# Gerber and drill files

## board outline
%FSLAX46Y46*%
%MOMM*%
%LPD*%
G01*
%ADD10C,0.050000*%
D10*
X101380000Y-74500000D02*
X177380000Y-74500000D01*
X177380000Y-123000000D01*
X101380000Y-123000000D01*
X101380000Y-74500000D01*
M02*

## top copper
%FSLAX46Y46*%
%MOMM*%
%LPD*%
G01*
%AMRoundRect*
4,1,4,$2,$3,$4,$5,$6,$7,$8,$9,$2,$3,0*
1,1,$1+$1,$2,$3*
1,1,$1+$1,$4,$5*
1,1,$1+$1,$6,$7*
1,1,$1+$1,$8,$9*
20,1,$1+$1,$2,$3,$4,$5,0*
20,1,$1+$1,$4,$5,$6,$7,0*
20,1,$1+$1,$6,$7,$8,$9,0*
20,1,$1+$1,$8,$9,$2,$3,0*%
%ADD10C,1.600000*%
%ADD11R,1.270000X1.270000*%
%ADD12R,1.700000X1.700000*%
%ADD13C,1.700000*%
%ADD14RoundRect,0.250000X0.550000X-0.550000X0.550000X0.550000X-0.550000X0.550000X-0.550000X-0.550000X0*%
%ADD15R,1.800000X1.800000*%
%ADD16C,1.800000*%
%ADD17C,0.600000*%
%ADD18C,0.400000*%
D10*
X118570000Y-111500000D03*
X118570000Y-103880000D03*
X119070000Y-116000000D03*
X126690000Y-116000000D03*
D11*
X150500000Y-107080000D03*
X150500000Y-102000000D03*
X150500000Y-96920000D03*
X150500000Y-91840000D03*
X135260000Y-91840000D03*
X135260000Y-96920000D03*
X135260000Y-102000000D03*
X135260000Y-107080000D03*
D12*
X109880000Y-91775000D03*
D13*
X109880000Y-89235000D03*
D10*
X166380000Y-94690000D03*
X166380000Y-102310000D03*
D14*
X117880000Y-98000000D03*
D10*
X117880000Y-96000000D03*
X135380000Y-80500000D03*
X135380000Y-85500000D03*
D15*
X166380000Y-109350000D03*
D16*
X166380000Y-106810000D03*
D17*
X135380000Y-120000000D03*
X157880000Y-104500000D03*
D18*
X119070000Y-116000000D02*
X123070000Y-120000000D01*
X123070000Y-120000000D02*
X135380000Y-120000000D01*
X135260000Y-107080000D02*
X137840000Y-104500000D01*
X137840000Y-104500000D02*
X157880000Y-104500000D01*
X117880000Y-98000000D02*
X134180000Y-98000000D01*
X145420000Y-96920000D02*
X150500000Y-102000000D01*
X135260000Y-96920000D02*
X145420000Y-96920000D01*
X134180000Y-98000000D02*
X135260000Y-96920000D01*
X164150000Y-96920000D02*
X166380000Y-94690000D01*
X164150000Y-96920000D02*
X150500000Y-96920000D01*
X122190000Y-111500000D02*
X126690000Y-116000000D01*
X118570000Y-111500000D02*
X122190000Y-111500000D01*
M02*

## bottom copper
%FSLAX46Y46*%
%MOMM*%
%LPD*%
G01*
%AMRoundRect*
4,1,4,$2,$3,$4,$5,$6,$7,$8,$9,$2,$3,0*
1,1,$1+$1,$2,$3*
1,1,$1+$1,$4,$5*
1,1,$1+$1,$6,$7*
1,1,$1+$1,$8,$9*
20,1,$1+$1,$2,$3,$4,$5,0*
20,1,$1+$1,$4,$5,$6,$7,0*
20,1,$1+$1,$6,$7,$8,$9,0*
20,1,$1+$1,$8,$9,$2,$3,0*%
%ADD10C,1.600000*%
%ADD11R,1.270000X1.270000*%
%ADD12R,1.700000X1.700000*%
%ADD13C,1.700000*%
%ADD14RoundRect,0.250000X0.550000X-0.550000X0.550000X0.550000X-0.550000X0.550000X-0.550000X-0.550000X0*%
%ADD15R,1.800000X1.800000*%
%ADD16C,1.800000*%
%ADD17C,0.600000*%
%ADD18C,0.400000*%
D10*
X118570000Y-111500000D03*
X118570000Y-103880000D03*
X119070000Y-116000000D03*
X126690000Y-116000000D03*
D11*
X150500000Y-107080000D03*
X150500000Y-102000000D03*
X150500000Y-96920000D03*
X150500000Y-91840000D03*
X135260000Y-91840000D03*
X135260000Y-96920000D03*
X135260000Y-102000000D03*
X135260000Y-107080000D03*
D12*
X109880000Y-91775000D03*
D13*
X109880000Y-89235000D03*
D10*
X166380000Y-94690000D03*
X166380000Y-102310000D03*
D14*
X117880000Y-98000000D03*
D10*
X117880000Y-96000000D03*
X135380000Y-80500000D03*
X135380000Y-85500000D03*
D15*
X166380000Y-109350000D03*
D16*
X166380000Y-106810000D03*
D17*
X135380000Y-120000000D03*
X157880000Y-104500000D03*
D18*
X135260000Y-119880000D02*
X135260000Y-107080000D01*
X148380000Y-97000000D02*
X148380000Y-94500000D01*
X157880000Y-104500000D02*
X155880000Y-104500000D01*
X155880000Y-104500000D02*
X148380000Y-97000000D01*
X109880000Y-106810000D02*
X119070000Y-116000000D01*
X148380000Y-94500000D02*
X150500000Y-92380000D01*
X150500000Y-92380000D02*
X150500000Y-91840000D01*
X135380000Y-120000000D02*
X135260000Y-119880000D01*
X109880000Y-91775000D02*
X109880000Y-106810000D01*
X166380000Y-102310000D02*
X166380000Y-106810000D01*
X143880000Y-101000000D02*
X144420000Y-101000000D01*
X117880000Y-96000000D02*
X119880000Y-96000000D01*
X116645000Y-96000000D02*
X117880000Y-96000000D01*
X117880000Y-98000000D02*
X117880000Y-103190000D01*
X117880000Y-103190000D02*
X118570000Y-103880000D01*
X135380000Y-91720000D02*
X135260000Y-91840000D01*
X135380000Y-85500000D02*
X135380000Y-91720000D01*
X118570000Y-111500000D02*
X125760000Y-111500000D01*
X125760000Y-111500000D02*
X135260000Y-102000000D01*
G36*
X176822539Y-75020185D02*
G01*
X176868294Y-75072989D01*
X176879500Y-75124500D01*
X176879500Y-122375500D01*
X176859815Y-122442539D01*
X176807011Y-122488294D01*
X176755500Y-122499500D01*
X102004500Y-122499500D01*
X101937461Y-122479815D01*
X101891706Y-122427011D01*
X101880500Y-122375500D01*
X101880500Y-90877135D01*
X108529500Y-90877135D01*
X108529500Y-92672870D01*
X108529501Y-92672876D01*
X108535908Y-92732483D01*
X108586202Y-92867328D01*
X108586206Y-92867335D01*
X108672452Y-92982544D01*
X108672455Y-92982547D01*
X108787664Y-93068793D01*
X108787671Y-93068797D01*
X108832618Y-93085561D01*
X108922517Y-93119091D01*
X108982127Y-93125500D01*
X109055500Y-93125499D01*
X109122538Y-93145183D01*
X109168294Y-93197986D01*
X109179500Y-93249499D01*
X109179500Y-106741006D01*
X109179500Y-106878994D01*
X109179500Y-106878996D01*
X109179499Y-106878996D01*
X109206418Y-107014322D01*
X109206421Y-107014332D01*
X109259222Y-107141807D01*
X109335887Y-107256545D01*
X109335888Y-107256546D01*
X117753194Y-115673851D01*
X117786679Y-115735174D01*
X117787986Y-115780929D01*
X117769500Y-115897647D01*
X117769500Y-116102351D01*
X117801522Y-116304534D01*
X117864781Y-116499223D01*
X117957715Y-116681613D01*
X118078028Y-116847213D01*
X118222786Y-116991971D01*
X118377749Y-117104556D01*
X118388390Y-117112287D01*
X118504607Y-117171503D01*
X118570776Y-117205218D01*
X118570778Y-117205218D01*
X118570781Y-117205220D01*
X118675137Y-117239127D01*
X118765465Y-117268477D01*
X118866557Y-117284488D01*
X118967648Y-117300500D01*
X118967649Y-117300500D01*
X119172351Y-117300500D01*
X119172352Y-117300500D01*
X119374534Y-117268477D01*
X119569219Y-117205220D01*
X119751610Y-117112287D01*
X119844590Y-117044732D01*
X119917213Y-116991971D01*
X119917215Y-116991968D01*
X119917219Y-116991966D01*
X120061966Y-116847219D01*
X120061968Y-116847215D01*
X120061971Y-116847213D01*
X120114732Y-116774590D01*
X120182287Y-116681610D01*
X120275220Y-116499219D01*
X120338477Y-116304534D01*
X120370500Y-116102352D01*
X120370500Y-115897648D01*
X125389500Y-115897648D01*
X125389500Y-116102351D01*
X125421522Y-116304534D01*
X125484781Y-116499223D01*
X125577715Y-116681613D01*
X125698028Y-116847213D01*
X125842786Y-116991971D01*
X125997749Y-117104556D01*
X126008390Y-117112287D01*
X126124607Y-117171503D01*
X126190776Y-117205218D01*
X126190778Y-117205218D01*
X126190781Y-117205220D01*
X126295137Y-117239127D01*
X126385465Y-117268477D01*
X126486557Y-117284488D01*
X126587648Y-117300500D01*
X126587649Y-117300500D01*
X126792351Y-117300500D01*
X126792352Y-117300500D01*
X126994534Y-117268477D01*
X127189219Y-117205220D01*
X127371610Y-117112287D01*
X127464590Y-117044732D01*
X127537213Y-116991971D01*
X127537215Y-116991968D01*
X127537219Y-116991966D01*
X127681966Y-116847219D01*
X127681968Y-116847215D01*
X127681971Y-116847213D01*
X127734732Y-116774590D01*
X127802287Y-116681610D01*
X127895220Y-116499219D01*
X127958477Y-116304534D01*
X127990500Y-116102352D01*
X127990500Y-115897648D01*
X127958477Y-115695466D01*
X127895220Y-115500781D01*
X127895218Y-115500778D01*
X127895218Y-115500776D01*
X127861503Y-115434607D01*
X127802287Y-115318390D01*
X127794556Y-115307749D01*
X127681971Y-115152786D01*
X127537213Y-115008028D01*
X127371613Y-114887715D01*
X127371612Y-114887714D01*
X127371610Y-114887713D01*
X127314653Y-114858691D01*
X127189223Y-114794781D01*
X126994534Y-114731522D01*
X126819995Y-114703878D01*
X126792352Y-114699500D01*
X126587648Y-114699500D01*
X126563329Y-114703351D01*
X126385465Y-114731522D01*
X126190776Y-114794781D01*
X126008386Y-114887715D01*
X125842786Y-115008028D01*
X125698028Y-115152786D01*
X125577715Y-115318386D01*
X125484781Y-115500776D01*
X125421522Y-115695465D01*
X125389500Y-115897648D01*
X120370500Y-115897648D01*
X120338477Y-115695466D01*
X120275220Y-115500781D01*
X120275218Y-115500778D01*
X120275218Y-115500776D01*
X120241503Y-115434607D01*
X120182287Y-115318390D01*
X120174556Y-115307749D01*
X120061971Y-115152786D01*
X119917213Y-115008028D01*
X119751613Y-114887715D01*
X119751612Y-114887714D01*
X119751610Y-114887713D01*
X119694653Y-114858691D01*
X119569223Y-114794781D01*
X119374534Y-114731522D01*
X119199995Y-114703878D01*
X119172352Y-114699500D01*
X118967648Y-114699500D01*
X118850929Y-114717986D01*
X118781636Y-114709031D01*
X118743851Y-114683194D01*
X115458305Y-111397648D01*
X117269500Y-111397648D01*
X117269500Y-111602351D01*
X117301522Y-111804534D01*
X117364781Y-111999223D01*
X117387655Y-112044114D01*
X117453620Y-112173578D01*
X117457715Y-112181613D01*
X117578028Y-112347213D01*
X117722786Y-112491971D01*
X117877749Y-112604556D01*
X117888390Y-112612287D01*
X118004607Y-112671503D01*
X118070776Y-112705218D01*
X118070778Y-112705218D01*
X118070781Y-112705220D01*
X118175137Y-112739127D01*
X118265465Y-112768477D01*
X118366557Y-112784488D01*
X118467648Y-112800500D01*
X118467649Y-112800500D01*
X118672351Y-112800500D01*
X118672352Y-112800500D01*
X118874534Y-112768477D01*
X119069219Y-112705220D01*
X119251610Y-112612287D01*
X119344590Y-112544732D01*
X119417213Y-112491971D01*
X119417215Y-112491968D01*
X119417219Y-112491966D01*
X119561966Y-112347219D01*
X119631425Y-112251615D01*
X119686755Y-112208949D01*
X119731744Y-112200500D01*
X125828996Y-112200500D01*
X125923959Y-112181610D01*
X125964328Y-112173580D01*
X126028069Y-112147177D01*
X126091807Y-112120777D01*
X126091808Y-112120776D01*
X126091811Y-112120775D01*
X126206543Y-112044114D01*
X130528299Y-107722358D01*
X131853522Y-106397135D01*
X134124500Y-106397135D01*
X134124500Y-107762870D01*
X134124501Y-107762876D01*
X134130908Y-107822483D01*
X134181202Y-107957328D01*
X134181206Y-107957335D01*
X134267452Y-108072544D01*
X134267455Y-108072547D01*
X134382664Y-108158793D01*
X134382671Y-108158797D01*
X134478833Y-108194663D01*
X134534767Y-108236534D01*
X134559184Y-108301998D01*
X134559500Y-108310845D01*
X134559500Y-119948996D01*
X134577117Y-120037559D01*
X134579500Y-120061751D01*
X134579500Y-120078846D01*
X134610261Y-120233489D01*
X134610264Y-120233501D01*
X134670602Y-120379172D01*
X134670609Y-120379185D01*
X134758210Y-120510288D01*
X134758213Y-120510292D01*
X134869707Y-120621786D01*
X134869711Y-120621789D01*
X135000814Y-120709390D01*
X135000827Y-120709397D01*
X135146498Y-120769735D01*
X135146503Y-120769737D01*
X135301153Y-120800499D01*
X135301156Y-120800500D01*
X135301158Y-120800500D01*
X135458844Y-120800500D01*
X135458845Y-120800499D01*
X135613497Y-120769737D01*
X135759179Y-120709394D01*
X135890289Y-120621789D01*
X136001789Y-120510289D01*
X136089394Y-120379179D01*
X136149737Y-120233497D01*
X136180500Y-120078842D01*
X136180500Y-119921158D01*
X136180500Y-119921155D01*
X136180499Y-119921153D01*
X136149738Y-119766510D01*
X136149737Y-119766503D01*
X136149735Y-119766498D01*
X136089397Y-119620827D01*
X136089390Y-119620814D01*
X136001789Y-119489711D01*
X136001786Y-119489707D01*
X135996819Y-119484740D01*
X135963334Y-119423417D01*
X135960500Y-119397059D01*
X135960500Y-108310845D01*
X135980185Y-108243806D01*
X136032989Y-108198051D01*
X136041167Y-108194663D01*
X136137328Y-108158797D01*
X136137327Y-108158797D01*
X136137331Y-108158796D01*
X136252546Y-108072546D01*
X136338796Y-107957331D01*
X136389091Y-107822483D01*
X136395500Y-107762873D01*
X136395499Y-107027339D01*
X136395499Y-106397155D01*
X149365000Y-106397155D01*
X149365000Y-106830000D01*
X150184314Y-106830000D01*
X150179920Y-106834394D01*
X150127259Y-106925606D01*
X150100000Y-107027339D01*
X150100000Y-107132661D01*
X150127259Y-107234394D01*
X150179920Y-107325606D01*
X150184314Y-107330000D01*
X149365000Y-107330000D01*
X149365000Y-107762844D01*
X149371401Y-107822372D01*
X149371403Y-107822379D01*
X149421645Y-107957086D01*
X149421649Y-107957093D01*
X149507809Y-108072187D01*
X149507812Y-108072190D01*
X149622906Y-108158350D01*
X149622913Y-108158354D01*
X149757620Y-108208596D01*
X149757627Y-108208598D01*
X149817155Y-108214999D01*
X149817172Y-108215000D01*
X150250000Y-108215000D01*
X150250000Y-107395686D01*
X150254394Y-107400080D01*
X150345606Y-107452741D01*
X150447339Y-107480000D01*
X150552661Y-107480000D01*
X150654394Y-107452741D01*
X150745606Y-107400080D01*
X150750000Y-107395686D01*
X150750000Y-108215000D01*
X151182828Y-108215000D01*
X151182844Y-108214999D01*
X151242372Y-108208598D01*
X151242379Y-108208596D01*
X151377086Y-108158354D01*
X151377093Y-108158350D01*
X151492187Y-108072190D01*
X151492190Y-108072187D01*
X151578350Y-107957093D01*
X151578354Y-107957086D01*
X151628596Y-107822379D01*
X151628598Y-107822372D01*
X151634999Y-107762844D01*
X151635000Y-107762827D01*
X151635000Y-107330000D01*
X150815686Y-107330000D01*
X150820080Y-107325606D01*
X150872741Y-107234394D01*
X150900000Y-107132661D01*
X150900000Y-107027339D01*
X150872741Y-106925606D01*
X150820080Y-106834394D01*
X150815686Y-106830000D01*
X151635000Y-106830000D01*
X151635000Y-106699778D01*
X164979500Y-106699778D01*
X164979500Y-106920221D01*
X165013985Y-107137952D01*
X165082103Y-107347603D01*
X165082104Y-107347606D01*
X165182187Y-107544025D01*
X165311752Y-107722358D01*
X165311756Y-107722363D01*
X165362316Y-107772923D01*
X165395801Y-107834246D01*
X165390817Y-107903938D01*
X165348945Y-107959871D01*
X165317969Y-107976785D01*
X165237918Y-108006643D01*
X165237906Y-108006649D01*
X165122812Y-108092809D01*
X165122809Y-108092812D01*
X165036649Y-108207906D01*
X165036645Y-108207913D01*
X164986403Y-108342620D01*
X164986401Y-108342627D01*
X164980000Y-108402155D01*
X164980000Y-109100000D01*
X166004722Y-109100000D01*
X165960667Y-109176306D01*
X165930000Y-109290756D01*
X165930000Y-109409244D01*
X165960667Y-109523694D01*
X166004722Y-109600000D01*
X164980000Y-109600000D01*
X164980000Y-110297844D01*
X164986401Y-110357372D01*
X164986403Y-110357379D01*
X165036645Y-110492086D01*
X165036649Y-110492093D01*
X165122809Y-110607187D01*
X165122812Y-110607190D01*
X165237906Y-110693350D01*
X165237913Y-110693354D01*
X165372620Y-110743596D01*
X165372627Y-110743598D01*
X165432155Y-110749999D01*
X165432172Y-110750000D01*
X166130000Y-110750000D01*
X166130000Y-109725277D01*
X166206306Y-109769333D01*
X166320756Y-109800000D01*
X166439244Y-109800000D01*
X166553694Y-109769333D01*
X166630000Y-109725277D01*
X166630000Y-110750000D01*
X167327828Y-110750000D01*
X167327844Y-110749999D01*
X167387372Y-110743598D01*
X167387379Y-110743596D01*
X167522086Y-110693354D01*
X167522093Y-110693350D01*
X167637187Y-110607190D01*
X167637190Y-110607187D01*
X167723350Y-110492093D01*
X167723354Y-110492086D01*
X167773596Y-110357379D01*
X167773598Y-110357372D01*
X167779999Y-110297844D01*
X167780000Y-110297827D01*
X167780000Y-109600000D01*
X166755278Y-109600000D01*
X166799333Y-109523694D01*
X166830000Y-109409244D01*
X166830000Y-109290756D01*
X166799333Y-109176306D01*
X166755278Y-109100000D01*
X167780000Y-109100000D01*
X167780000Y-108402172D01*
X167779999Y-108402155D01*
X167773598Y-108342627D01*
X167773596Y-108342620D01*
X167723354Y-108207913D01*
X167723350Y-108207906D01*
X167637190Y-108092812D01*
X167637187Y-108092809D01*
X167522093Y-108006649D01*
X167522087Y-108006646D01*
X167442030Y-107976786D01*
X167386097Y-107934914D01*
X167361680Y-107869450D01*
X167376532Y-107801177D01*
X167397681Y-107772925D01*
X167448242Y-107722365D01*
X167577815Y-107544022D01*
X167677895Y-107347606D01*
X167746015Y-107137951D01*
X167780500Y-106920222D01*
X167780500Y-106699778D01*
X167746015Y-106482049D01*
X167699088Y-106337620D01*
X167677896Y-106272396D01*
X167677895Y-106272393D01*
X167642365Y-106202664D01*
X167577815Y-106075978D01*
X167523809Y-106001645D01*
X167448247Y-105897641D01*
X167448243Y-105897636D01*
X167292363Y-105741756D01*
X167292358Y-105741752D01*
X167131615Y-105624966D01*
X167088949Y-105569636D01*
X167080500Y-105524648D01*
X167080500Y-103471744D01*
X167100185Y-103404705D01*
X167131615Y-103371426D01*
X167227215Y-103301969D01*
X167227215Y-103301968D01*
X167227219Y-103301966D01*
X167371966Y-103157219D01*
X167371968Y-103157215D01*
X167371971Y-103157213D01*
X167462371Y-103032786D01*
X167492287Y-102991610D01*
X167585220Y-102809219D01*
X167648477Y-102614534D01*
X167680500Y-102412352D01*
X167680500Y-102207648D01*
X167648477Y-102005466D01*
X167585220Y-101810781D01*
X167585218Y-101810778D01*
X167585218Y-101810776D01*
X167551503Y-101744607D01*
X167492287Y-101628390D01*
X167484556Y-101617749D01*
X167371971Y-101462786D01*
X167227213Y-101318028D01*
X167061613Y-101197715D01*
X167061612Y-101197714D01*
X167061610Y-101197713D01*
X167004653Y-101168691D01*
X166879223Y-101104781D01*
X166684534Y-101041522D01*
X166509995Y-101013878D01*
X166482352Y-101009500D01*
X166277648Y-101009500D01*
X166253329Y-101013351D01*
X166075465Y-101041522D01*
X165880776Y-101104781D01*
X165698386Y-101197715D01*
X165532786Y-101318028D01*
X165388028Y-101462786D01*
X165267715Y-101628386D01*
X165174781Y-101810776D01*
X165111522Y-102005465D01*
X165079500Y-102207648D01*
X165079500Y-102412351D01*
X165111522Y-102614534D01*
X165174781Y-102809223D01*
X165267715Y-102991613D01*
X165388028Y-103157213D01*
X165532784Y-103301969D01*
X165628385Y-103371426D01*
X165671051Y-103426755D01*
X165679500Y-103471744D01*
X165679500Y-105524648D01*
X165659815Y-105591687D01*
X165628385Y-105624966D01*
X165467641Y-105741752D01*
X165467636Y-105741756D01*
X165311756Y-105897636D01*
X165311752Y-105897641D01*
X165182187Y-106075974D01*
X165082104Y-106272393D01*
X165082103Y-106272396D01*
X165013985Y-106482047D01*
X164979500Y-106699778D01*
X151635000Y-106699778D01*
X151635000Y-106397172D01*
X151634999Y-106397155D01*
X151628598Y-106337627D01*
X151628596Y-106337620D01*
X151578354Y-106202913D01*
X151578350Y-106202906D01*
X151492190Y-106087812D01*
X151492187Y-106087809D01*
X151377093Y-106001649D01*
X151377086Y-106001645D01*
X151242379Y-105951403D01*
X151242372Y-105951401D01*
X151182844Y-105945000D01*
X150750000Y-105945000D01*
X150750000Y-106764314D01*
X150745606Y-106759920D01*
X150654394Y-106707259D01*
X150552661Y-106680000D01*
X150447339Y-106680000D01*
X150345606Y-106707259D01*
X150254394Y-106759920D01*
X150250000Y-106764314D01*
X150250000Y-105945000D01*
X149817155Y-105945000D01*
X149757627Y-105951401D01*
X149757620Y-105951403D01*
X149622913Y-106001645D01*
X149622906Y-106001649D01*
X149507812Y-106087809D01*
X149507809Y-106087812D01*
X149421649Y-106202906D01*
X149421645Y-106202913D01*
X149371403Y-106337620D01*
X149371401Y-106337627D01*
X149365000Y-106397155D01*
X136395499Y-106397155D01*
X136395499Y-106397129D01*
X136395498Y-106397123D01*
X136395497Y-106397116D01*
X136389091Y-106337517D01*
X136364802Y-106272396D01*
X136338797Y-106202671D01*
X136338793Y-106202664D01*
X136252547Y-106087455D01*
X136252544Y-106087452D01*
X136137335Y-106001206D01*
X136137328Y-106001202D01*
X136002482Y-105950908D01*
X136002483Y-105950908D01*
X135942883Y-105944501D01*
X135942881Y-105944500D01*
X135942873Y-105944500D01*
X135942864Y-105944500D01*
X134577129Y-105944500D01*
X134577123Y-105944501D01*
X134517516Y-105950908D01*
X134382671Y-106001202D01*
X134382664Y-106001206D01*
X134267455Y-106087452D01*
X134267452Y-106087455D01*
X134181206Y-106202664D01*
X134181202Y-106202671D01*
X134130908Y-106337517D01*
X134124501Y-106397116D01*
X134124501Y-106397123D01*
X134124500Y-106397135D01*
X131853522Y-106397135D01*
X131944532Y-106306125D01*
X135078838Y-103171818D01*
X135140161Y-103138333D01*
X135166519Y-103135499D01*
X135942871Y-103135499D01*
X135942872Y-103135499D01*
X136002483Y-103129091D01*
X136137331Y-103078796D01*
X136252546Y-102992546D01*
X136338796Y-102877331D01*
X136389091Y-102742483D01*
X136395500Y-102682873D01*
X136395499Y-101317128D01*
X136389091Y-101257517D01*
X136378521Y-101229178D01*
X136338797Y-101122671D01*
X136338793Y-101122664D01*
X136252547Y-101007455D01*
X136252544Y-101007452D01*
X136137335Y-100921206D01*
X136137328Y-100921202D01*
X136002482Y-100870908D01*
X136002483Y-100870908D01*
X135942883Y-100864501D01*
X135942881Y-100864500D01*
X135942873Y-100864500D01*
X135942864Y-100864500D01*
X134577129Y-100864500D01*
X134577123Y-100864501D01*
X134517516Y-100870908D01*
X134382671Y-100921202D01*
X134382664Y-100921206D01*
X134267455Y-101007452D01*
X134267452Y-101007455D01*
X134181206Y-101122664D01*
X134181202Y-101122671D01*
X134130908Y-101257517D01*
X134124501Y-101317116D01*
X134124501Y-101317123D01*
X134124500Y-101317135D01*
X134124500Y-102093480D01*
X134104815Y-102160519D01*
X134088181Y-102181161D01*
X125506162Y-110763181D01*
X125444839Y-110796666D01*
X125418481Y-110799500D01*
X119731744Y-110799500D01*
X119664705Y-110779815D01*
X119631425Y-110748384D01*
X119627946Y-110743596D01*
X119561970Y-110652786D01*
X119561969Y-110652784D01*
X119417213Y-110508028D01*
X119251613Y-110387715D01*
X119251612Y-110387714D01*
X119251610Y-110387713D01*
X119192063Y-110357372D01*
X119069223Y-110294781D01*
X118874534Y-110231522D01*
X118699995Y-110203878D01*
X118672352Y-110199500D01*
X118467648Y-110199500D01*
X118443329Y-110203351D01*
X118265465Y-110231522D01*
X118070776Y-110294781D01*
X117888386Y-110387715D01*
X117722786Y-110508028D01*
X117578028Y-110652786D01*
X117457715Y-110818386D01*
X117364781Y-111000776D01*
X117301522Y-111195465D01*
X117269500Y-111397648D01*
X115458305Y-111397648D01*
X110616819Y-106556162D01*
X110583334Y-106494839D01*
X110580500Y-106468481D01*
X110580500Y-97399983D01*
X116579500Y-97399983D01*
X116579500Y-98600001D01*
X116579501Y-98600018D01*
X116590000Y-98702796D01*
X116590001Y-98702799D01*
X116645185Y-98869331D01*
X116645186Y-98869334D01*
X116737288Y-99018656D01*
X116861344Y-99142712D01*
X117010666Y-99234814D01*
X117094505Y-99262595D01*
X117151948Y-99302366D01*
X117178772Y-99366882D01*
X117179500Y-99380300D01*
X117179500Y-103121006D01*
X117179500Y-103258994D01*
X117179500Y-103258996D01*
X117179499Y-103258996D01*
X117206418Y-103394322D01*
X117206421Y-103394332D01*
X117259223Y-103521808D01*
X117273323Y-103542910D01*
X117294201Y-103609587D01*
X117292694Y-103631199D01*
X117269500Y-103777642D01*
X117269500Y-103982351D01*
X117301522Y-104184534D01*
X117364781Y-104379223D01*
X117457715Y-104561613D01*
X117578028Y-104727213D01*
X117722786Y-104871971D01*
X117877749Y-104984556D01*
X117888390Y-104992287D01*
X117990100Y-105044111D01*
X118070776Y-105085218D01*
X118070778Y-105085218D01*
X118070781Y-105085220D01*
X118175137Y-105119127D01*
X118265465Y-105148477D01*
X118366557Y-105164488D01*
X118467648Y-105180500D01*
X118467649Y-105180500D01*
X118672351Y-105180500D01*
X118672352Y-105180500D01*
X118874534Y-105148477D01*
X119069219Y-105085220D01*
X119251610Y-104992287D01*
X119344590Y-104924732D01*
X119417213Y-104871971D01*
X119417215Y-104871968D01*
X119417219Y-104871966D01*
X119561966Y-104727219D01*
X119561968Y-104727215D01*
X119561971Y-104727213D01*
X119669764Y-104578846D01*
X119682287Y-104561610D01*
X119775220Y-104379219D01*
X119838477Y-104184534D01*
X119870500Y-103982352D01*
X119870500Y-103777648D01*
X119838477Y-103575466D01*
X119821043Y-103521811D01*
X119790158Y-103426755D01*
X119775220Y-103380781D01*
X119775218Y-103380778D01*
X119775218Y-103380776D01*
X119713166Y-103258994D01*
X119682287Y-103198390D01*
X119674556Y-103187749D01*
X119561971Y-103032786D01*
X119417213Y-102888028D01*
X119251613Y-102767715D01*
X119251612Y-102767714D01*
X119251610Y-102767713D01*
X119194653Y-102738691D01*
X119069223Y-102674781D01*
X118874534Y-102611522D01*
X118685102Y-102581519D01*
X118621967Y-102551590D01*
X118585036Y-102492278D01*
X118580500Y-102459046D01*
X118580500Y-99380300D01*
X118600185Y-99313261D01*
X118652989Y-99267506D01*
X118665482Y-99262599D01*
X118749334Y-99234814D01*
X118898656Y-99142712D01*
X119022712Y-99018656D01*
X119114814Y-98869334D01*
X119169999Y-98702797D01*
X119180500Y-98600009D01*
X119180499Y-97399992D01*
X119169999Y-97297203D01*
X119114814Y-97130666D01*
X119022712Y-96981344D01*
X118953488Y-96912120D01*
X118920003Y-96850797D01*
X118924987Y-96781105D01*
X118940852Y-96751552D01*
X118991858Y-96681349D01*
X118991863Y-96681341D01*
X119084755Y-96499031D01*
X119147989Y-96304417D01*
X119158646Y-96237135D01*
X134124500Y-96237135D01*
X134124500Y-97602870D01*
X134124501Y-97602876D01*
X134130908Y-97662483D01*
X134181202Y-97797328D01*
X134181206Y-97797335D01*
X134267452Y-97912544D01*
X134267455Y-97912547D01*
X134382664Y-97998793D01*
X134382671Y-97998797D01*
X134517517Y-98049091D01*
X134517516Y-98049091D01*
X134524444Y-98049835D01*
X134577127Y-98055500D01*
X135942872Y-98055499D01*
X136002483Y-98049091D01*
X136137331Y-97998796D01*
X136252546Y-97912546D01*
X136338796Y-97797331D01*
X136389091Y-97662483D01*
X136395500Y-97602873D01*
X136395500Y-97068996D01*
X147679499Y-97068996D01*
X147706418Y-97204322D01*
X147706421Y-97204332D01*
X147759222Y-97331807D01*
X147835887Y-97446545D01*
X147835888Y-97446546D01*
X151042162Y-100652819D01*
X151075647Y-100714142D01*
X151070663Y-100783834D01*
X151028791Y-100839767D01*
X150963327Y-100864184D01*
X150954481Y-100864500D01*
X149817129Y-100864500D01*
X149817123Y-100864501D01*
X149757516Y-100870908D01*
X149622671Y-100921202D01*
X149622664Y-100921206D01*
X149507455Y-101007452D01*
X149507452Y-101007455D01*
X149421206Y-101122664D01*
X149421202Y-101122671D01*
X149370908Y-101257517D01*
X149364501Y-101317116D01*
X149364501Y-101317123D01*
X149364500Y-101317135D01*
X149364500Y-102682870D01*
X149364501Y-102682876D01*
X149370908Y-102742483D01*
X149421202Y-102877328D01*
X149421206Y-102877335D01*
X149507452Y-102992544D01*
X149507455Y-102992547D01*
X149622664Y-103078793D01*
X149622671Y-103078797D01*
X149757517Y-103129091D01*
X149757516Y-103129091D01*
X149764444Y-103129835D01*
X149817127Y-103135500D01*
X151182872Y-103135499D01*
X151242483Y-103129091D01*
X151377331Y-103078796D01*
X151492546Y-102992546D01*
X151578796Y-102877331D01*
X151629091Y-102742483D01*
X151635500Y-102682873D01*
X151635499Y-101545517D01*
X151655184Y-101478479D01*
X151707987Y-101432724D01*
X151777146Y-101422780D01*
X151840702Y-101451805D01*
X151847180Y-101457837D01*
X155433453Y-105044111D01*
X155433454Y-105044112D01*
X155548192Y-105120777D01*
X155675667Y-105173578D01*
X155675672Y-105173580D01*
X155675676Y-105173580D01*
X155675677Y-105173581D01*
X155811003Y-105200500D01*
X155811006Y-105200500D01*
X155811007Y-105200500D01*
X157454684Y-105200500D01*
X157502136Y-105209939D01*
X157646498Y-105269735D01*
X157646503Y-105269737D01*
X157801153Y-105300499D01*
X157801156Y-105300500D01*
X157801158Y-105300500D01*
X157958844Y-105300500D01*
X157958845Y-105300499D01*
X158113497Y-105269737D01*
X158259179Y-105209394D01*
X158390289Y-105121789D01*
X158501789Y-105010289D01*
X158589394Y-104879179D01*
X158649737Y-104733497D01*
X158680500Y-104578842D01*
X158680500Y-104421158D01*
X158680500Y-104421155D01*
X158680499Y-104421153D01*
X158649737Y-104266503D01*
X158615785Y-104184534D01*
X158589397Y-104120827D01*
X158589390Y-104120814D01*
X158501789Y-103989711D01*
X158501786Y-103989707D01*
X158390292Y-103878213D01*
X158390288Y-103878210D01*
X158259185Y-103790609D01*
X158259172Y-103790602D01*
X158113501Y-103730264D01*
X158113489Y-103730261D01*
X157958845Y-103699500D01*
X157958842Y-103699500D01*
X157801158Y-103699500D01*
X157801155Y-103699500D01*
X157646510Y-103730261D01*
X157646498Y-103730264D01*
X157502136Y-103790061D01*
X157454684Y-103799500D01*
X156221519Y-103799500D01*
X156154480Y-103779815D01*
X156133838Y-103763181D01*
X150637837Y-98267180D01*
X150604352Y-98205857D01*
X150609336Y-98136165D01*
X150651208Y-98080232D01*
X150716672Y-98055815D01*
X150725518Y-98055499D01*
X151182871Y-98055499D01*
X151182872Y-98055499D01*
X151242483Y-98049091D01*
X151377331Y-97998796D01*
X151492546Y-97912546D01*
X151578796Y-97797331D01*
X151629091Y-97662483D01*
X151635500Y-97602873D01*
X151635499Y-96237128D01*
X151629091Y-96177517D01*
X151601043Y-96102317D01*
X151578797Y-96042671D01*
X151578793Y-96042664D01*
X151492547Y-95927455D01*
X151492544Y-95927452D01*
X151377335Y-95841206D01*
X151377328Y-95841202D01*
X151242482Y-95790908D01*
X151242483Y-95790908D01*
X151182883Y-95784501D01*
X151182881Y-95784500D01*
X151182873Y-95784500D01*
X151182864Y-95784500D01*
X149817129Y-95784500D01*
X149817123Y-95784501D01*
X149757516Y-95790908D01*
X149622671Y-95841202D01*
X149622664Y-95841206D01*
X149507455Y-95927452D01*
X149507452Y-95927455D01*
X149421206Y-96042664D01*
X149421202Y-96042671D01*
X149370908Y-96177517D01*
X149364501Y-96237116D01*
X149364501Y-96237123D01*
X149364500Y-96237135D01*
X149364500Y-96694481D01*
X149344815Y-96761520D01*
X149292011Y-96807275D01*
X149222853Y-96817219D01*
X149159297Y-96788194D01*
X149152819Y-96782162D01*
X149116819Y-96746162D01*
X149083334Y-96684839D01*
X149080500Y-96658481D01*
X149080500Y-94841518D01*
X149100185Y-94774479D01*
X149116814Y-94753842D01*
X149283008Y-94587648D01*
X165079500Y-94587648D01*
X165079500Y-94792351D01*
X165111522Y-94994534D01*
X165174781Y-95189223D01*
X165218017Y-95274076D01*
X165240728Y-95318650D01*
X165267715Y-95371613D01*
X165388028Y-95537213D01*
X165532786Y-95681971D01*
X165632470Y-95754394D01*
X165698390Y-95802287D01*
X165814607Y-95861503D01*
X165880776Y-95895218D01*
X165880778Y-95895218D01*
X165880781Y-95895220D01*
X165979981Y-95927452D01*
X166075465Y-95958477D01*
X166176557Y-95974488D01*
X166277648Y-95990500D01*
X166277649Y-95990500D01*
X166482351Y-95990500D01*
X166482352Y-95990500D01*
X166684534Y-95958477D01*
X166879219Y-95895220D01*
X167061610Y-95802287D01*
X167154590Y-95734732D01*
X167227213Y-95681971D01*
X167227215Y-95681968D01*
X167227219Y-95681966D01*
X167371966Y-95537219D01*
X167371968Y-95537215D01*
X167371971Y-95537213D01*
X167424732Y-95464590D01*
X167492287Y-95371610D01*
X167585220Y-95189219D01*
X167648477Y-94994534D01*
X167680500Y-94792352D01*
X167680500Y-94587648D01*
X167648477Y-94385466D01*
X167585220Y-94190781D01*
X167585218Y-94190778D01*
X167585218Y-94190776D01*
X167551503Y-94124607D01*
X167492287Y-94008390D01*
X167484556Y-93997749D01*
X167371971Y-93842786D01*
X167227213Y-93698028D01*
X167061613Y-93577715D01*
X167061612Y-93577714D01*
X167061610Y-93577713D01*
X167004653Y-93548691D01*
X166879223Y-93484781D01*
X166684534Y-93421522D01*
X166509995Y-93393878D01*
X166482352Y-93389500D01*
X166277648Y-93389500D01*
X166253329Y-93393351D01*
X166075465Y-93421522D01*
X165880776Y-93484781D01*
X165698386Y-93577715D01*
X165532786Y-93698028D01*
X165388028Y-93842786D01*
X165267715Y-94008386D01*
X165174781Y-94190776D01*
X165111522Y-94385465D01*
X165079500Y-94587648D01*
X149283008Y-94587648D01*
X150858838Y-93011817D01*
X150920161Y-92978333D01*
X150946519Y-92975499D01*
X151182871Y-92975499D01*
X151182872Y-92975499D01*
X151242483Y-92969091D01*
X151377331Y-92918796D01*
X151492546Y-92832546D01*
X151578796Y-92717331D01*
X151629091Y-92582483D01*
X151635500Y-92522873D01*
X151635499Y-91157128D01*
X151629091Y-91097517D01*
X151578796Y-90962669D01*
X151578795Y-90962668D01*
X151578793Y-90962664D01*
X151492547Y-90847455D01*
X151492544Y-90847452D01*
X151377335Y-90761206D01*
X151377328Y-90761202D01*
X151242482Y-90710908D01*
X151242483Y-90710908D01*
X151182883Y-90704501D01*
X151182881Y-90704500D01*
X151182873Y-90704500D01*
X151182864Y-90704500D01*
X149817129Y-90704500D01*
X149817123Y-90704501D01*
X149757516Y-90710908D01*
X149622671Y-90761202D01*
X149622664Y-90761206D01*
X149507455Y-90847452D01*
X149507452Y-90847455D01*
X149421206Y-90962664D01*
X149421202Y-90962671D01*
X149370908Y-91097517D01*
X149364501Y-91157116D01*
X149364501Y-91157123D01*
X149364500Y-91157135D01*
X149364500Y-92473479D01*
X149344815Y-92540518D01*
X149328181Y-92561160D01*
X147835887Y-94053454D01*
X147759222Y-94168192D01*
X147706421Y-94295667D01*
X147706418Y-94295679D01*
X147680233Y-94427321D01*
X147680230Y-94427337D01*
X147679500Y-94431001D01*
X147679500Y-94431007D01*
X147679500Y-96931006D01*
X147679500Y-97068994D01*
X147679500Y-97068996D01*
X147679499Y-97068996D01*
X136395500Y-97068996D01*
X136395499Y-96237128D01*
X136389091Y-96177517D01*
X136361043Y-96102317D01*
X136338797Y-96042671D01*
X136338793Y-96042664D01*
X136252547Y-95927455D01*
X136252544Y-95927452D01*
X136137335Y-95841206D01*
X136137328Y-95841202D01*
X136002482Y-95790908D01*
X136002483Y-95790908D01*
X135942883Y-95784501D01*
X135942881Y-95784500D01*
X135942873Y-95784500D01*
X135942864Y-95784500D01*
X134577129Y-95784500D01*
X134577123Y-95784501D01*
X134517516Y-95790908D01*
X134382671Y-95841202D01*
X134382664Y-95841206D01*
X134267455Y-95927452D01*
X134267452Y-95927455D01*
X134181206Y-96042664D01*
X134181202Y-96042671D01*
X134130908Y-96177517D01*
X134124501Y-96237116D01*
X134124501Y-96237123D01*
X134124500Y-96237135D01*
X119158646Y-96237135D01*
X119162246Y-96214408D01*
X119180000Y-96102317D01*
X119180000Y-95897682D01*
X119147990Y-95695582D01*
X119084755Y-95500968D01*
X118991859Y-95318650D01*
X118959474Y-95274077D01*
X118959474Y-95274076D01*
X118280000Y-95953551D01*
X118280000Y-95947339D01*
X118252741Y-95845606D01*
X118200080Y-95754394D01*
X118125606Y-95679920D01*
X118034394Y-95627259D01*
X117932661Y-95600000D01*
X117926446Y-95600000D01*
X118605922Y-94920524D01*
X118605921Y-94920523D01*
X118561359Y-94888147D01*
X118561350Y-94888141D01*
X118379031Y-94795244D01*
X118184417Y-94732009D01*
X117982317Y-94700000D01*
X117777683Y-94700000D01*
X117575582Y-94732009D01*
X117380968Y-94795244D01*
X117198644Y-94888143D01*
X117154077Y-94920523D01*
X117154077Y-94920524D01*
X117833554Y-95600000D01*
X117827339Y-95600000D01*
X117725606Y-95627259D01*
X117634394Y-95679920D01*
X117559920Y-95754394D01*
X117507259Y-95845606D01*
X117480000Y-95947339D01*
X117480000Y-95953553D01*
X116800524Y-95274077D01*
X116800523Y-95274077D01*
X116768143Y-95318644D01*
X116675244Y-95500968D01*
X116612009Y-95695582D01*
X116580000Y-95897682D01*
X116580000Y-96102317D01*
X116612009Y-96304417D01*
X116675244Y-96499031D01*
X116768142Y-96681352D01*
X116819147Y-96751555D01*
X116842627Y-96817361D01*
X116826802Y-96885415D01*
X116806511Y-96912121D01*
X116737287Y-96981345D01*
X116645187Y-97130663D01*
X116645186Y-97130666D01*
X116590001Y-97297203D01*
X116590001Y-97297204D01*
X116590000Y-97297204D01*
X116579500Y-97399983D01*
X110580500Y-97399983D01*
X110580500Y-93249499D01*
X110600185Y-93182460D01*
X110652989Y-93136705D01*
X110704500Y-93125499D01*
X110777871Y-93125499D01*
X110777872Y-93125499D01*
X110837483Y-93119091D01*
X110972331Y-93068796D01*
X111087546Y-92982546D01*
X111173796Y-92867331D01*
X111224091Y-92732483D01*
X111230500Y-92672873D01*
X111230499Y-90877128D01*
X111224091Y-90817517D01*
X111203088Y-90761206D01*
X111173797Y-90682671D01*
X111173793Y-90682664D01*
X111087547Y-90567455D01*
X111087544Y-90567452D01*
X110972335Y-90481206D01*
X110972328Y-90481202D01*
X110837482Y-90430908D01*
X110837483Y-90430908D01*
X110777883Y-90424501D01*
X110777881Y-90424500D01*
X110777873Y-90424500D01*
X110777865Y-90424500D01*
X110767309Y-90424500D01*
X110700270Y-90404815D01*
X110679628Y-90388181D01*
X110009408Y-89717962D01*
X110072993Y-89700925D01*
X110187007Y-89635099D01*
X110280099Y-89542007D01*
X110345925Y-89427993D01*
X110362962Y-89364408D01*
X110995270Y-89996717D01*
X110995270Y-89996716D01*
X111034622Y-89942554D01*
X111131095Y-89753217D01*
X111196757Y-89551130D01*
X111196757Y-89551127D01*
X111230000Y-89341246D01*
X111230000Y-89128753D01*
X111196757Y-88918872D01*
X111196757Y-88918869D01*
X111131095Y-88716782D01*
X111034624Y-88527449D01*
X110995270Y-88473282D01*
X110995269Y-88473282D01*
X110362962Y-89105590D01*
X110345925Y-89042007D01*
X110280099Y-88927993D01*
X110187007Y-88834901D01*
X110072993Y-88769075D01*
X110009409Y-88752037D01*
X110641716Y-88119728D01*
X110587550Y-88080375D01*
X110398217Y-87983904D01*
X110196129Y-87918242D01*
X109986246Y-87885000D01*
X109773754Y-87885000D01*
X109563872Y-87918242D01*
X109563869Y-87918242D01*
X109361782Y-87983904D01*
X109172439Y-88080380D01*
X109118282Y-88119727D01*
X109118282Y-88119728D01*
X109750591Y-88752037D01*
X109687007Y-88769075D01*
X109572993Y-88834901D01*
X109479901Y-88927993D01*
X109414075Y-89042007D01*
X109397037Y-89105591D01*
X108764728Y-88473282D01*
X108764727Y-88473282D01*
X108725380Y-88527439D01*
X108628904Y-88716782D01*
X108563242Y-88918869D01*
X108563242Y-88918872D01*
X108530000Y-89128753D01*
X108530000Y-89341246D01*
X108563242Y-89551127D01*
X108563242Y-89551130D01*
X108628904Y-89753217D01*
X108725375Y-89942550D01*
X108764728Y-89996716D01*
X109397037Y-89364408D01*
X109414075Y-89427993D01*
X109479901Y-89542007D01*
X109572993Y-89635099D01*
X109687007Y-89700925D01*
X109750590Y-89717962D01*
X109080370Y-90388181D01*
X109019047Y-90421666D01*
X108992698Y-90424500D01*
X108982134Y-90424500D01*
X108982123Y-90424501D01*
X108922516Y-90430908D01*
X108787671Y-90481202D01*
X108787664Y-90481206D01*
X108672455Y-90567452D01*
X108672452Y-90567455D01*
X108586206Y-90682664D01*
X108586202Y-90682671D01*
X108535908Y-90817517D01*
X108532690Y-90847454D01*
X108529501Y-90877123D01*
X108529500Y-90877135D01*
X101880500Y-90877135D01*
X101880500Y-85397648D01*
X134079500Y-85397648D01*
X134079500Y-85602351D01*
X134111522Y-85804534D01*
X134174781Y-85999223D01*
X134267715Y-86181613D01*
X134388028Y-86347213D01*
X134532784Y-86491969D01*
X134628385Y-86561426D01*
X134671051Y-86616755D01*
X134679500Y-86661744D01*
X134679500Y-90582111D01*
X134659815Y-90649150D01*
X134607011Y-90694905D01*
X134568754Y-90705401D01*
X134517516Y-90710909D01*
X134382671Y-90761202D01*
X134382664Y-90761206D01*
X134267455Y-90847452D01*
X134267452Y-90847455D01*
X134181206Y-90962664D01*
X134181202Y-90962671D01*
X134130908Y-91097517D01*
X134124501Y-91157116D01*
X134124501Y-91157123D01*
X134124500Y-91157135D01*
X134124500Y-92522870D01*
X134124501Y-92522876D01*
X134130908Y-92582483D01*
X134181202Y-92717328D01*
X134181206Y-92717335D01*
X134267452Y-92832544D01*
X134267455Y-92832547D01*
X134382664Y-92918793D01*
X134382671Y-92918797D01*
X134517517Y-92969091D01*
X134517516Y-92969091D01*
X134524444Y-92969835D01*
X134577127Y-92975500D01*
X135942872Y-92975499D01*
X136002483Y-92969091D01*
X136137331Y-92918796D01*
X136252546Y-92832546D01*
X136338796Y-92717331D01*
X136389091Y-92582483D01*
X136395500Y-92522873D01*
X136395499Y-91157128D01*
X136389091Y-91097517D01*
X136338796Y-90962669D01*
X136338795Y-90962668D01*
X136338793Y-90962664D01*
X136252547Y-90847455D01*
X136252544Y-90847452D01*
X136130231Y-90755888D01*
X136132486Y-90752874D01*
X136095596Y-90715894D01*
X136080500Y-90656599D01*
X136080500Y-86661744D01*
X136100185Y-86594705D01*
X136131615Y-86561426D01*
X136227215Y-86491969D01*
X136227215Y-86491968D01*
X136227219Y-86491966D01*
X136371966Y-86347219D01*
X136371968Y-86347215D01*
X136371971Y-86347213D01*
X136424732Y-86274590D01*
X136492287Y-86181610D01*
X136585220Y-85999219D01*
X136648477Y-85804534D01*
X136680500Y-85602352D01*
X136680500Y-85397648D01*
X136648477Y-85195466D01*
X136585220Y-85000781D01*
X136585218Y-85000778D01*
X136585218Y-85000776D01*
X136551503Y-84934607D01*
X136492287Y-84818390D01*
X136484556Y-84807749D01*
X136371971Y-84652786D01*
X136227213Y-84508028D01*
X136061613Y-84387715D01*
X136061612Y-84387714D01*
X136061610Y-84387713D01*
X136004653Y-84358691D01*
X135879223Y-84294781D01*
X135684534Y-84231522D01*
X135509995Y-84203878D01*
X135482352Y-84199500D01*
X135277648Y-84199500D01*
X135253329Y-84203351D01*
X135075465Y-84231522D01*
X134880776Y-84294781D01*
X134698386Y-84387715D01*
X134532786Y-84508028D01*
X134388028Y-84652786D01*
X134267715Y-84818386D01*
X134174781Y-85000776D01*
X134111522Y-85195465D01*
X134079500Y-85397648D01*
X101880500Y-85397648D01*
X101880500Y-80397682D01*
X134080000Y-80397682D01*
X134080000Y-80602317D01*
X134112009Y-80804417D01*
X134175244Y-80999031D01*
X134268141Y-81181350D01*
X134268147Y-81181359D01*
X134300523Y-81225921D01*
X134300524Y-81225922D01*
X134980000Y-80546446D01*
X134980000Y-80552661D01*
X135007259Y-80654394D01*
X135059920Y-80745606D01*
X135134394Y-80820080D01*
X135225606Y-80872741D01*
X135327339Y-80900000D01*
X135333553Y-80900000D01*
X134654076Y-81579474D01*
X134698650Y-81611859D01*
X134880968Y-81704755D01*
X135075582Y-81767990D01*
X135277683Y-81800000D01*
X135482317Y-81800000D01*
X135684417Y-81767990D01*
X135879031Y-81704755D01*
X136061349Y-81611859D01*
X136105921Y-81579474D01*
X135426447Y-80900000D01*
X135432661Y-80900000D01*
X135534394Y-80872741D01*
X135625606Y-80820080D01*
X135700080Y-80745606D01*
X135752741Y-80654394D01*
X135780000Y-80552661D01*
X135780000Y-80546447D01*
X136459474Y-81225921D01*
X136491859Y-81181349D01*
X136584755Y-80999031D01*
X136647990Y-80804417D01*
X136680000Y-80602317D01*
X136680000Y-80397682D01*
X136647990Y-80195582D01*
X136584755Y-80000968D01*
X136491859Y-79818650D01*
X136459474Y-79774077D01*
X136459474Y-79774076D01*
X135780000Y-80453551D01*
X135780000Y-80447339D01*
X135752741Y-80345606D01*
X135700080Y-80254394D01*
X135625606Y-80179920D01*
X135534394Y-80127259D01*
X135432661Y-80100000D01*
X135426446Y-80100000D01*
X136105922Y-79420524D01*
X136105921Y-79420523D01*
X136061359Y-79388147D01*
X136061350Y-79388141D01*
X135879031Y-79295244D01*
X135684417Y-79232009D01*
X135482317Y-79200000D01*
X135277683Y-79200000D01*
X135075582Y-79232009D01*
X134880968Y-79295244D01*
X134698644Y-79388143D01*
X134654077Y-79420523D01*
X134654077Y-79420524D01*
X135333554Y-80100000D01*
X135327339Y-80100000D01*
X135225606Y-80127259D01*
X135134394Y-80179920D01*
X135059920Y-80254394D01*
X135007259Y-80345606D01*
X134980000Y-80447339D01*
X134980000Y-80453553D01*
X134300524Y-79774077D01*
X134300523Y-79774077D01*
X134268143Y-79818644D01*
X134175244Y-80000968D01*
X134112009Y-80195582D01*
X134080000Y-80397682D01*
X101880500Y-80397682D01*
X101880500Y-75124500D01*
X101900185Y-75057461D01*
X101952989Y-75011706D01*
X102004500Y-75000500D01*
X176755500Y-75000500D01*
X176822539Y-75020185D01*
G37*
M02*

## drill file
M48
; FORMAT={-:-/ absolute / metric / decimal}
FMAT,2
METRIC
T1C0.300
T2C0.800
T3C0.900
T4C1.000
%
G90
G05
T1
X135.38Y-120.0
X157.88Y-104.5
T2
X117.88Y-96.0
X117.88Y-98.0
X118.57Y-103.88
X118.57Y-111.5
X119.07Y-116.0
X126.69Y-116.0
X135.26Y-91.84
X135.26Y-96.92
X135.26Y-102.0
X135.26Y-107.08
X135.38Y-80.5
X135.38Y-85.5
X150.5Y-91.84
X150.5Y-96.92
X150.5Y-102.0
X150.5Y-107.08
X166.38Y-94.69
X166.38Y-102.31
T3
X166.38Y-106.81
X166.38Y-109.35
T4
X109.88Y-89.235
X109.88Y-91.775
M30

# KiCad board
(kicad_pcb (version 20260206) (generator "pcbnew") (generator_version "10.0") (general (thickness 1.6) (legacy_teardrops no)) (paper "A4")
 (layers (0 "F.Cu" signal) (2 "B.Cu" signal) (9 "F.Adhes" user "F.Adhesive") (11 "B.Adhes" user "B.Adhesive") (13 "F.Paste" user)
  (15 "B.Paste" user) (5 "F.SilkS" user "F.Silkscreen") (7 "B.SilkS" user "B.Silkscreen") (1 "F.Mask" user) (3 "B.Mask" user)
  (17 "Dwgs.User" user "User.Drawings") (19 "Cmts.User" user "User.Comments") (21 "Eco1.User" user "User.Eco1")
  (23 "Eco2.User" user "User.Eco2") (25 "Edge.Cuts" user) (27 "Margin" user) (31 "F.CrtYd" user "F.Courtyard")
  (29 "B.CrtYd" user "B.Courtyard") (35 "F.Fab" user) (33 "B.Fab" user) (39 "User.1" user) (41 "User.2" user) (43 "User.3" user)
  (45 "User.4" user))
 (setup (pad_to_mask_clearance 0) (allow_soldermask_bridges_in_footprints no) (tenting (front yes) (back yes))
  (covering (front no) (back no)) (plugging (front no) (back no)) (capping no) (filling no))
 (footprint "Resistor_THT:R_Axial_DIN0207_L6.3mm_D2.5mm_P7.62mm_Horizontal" (layer "F.Cu") (at 118.57 111.5 90)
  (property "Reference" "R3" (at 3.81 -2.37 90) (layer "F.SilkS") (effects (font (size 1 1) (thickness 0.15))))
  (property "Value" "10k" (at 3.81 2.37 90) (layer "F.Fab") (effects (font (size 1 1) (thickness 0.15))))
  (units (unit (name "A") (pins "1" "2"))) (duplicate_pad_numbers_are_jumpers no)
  (pad "1" thru_hole circle (at 0 0 90) (size 1.6 1.6) (drill 0.8) (layers "*.Cu" "*.Mask") (remove_unused_layers no) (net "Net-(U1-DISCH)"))
  (pad "2" thru_hole circle (at 7.62 0 90) (size 1.6 1.6) (drill 0.8) (layers "*.Cu" "*.Mask") (remove_unused_layers no)
   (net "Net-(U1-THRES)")))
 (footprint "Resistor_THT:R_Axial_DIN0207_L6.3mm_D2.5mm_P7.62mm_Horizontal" (layer "F.Cu") (at 119.07 116)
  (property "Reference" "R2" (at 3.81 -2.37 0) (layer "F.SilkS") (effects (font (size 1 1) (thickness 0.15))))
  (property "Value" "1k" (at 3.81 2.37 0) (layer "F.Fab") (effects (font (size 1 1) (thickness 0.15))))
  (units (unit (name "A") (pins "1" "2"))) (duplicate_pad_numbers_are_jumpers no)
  (pad "1" thru_hole circle (at 0 0) (size 1.6 1.6) (drill 0.8) (layers "*.Cu" "*.Mask") (remove_unused_layers no) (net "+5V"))
  (pad "2" thru_hole circle (at 7.62 0) (size 1.6 1.6) (drill 0.8) (layers "*.Cu" "*.Mask") (remove_unused_layers no) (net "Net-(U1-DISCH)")))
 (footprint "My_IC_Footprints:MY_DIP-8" (layer "F.Cu") (at 142.88 102 180)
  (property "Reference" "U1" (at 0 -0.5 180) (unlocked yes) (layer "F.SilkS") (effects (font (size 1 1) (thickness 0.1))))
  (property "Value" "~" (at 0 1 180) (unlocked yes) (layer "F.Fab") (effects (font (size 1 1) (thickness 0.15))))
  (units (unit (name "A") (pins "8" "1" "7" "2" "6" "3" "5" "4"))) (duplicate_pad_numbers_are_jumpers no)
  (pad "1" thru_hole rect (at -7.62 -5.08 180) (size 1.27 1.27) (drill 0.8) (layers "*.Cu" "*.Mask") (remove_unused_layers no) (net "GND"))
  (pad "2" thru_hole rect (at -7.62 0 180) (size 1.27 1.27) (drill 0.8) (layers "*.Cu" "*.Mask") (remove_unused_layers no)
   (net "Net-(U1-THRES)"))
  (pad "3" thru_hole rect (at -7.62 5.08 180) (size 1.27 1.27) (drill 0.8) (layers "*.Cu" "*.Mask") (remove_unused_layers no)
   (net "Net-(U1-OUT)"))
  (pad "4" thru_hole rect (at -7.62 10.16 180) (size 1.27 1.27) (drill 0.8) (layers "*.Cu" "*.Mask") (remove_unused_layers no) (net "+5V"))
  (pad "5" thru_hole rect (at 7.62 10.16 180) (size 1.27 1.27) (drill 0.8) (layers "*.Cu" "*.Mask") (remove_unused_layers no)
   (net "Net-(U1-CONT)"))
  (pad "6" thru_hole rect (at 7.62 5.08 180) (size 1.27 1.27) (drill 0.8) (layers "*.Cu" "*.Mask") (remove_unused_layers no)
   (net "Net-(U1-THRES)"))
  (pad "7" thru_hole rect (at 7.62 0 180) (size 1.27 1.27) (drill 0.8) (layers "*.Cu" "*.Mask") (remove_unused_layers no)
   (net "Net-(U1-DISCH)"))
  (pad "8" thru_hole rect (at 7.62 -5.08 180) (size 1.27 1.27) (drill 0.8) (layers "*.Cu" "*.Mask") (remove_unused_layers no) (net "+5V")))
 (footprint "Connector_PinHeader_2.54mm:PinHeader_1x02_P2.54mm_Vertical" (layer "F.Cu") (at 109.88 91.775 180)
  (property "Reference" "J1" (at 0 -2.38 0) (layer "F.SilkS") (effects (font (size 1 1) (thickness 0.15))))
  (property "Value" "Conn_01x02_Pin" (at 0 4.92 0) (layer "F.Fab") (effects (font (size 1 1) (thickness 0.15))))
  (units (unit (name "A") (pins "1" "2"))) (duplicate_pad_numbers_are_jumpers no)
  (pad "1" thru_hole rect (at 0 0 180) (size 1.7 1.7) (drill 1) (layers "*.Cu" "*.Mask") (remove_unused_layers no) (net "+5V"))
  (pad "2" thru_hole circle (at 0 2.54 180) (size 1.7 1.7) (drill 1) (layers "*.Cu" "*.Mask") (remove_unused_layers no) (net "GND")))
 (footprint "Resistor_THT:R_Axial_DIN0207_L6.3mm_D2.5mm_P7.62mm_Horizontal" (layer "F.Cu") (at 166.38 94.69 -90)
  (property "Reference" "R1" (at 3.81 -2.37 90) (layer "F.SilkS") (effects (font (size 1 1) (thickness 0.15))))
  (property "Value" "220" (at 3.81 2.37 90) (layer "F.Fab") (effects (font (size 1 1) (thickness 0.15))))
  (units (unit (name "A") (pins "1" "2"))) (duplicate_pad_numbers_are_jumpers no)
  (pad "1" thru_hole circle (at 0 0 270) (size 1.6 1.6) (drill 0.8) (layers "*.Cu" "*.Mask") (remove_unused_layers no) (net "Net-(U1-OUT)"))
  (pad "2" thru_hole circle (at 7.62 0 270) (size 1.6 1.6) (drill 0.8) (layers "*.Cu" "*.Mask") (remove_unused_layers no) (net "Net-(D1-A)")))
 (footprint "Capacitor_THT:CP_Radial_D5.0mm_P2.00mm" (layer "F.Cu") (at 117.88 98 90)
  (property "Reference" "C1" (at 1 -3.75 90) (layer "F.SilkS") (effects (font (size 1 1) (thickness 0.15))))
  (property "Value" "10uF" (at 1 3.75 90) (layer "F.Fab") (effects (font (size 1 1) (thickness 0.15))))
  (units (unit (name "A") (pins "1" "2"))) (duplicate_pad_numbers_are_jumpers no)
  (pad "1" thru_hole roundrect (at 0 0 90) (size 1.6 1.6) (drill 0.8) (layers "*.Cu" "*.Mask") (remove_unused_layers no)
   (roundrect_rratio 0.15625) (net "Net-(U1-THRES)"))
  (pad "2" thru_hole circle (at 2 0 90) (size 1.6 1.6) (drill 0.8) (layers "*.Cu" "*.Mask") (remove_unused_layers no) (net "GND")))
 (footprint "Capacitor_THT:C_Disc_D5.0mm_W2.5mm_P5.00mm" (layer "F.Cu") (at 135.38 80.5 -90)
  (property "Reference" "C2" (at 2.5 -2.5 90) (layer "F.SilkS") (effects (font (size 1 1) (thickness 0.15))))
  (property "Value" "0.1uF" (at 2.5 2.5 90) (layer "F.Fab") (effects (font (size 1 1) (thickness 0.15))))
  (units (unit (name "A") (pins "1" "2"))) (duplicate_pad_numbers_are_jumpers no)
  (pad "1" thru_hole circle (at 0 0 270) (size 1.6 1.6) (drill 0.8) (layers "*.Cu" "*.Mask") (remove_unused_layers no) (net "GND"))
  (pad "2" thru_hole circle (at 5 0 270) (size 1.6 1.6) (drill 0.8) (layers "*.Cu" "*.Mask") (remove_unused_layers no) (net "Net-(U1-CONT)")))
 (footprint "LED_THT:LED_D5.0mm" (layer "F.Cu") (at 166.38 109.35 90)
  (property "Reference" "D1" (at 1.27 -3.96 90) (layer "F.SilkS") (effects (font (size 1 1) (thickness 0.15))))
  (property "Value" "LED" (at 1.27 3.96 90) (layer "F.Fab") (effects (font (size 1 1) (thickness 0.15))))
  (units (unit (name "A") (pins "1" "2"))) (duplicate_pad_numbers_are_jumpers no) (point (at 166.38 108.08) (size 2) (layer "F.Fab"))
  (pad "1" thru_hole rect (at 0 0 90) (size 1.8 1.8) (drill 0.9) (layers "*.Cu" "*.Mask") (remove_unused_layers no) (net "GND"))
  (pad "2" thru_hole circle (at 2.54 0 90) (size 1.8 1.8) (drill 0.9) (layers "*.Cu" "*.Mask") (remove_unused_layers no) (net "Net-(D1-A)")))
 (gr_rect (start 101.38 74.5) (end 177.38 123) (stroke (width 0.05) (type default)) (fill no) (layer "Edge.Cuts"))
 (segment (start 119.07 116) (end 123.07 120) (width 0.4) (layer "F.Cu") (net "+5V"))
 (segment (start 123.07 120) (end 135.38 120) (width 0.4) (layer "F.Cu") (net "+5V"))
 (segment (start 135.26 107.08) (end 137.84 104.5) (width 0.4) (layer "F.Cu") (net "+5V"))
 (segment (start 137.84 104.5) (end 157.88 104.5) (width 0.4) (layer "F.Cu") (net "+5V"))
 (via (at 135.38 120) (size 0.6) (drill 0.3) (layers "F.Cu" "B.Cu") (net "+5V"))
 (via (at 157.88 104.5) (size 0.6) (drill 0.3) (layers "F.Cu" "B.Cu") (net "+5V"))
 (segment (start 135.26 119.88) (end 135.26 107.08) (width 0.4) (layer "B.Cu") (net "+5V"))
 (segment (start 148.38 97) (end 148.38 94.5) (width 0.4) (layer "B.Cu") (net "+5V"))
 (segment (start 157.88 104.5) (end 155.88 104.5) (width 0.4) (layer "B.Cu") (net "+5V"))
 (segment (start 155.88 104.5) (end 148.38 97) (width 0.4) (layer "B.Cu") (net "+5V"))
 (segment (start 109.88 106.81) (end 119.07 116) (width 0.4) (layer "B.Cu") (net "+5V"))
 (segment (start 148.38 94.5) (end 150.5 92.38) (width 0.4) (layer "B.Cu") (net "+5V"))
 (segment (start 150.5 92.38) (end 150.5 91.84) (width 0.4) (layer "B.Cu") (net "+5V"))
 (segment (start 135.38 120) (end 135.26 119.88) (width 0.4) (layer "B.Cu") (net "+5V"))
 (segment (start 109.88 91.775) (end 109.88 106.81) (width 0.4) (layer "B.Cu") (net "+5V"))
 (segment (start 166.38 102.31) (end 166.38 106.81) (width 0.4) (layer "B.Cu") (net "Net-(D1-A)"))
 (segment (start 143.88 101) (end 144.42 101) (width 0.4) (layer "B.Cu") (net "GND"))
 (segment (start 117.88 96) (end 119.88 96) (width 0.4) (layer "B.Cu") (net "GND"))
 (segment (start 116.645 96) (end 117.88 96) (width 0.4) (layer "B.Cu") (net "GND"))
 (segment (start 117.88 98) (end 134.18 98) (width 0.4) (layer "F.Cu") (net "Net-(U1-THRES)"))
 (segment (start 145.42 96.92) (end 150.5 102) (width 0.4) (layer "F.Cu") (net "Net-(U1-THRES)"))
 (segment (start 135.26 96.92) (end 145.42 96.92) (width 0.4) (layer "F.Cu") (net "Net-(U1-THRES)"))
 (segment (start 134.18 98) (end 135.26 96.92) (width 0.4) (layer "F.Cu") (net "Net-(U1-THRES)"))
 (segment (start 117.88 98) (end 117.88 103.19) (width 0.4) (layer "B.Cu") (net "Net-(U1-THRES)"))
 (segment (start 117.88 103.19) (end 118.57 103.88) (width 0.4) (layer "B.Cu") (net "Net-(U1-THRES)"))
 (segment (start 135.38 91.72) (end 135.26 91.84) (width 0.4) (layer "B.Cu") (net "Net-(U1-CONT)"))
 (segment (start 135.38 85.5) (end 135.38 91.72) (width 0.4) (layer "B.Cu") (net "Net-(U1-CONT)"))
 (segment (start 164.15 96.92) (end 166.38 94.69) (width 0.4) (layer "F.Cu") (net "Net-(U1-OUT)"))
 (segment (start 164.15 96.92) (end 150.5 96.92) (width 0.4) (layer "F.Cu") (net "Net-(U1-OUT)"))
 (segment (start 122.19 111.5) (end 126.69 116) (width 0.4) (layer "F.Cu") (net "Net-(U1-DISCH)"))
 (segment (start 118.57 111.5) (end 122.19 111.5) (width 0.4) (layer "F.Cu") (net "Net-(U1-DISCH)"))
 (segment (start 118.57 111.5) (end 125.76 111.5) (width 0.4) (layer "B.Cu") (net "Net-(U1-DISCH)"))
 (segment (start 125.76 111.5) (end 135.26 102) (width 0.4) (layer "B.Cu") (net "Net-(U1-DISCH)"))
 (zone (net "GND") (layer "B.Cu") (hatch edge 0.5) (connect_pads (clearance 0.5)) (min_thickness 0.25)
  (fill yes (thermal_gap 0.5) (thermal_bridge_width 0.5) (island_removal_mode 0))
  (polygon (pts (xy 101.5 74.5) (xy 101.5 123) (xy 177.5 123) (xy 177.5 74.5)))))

